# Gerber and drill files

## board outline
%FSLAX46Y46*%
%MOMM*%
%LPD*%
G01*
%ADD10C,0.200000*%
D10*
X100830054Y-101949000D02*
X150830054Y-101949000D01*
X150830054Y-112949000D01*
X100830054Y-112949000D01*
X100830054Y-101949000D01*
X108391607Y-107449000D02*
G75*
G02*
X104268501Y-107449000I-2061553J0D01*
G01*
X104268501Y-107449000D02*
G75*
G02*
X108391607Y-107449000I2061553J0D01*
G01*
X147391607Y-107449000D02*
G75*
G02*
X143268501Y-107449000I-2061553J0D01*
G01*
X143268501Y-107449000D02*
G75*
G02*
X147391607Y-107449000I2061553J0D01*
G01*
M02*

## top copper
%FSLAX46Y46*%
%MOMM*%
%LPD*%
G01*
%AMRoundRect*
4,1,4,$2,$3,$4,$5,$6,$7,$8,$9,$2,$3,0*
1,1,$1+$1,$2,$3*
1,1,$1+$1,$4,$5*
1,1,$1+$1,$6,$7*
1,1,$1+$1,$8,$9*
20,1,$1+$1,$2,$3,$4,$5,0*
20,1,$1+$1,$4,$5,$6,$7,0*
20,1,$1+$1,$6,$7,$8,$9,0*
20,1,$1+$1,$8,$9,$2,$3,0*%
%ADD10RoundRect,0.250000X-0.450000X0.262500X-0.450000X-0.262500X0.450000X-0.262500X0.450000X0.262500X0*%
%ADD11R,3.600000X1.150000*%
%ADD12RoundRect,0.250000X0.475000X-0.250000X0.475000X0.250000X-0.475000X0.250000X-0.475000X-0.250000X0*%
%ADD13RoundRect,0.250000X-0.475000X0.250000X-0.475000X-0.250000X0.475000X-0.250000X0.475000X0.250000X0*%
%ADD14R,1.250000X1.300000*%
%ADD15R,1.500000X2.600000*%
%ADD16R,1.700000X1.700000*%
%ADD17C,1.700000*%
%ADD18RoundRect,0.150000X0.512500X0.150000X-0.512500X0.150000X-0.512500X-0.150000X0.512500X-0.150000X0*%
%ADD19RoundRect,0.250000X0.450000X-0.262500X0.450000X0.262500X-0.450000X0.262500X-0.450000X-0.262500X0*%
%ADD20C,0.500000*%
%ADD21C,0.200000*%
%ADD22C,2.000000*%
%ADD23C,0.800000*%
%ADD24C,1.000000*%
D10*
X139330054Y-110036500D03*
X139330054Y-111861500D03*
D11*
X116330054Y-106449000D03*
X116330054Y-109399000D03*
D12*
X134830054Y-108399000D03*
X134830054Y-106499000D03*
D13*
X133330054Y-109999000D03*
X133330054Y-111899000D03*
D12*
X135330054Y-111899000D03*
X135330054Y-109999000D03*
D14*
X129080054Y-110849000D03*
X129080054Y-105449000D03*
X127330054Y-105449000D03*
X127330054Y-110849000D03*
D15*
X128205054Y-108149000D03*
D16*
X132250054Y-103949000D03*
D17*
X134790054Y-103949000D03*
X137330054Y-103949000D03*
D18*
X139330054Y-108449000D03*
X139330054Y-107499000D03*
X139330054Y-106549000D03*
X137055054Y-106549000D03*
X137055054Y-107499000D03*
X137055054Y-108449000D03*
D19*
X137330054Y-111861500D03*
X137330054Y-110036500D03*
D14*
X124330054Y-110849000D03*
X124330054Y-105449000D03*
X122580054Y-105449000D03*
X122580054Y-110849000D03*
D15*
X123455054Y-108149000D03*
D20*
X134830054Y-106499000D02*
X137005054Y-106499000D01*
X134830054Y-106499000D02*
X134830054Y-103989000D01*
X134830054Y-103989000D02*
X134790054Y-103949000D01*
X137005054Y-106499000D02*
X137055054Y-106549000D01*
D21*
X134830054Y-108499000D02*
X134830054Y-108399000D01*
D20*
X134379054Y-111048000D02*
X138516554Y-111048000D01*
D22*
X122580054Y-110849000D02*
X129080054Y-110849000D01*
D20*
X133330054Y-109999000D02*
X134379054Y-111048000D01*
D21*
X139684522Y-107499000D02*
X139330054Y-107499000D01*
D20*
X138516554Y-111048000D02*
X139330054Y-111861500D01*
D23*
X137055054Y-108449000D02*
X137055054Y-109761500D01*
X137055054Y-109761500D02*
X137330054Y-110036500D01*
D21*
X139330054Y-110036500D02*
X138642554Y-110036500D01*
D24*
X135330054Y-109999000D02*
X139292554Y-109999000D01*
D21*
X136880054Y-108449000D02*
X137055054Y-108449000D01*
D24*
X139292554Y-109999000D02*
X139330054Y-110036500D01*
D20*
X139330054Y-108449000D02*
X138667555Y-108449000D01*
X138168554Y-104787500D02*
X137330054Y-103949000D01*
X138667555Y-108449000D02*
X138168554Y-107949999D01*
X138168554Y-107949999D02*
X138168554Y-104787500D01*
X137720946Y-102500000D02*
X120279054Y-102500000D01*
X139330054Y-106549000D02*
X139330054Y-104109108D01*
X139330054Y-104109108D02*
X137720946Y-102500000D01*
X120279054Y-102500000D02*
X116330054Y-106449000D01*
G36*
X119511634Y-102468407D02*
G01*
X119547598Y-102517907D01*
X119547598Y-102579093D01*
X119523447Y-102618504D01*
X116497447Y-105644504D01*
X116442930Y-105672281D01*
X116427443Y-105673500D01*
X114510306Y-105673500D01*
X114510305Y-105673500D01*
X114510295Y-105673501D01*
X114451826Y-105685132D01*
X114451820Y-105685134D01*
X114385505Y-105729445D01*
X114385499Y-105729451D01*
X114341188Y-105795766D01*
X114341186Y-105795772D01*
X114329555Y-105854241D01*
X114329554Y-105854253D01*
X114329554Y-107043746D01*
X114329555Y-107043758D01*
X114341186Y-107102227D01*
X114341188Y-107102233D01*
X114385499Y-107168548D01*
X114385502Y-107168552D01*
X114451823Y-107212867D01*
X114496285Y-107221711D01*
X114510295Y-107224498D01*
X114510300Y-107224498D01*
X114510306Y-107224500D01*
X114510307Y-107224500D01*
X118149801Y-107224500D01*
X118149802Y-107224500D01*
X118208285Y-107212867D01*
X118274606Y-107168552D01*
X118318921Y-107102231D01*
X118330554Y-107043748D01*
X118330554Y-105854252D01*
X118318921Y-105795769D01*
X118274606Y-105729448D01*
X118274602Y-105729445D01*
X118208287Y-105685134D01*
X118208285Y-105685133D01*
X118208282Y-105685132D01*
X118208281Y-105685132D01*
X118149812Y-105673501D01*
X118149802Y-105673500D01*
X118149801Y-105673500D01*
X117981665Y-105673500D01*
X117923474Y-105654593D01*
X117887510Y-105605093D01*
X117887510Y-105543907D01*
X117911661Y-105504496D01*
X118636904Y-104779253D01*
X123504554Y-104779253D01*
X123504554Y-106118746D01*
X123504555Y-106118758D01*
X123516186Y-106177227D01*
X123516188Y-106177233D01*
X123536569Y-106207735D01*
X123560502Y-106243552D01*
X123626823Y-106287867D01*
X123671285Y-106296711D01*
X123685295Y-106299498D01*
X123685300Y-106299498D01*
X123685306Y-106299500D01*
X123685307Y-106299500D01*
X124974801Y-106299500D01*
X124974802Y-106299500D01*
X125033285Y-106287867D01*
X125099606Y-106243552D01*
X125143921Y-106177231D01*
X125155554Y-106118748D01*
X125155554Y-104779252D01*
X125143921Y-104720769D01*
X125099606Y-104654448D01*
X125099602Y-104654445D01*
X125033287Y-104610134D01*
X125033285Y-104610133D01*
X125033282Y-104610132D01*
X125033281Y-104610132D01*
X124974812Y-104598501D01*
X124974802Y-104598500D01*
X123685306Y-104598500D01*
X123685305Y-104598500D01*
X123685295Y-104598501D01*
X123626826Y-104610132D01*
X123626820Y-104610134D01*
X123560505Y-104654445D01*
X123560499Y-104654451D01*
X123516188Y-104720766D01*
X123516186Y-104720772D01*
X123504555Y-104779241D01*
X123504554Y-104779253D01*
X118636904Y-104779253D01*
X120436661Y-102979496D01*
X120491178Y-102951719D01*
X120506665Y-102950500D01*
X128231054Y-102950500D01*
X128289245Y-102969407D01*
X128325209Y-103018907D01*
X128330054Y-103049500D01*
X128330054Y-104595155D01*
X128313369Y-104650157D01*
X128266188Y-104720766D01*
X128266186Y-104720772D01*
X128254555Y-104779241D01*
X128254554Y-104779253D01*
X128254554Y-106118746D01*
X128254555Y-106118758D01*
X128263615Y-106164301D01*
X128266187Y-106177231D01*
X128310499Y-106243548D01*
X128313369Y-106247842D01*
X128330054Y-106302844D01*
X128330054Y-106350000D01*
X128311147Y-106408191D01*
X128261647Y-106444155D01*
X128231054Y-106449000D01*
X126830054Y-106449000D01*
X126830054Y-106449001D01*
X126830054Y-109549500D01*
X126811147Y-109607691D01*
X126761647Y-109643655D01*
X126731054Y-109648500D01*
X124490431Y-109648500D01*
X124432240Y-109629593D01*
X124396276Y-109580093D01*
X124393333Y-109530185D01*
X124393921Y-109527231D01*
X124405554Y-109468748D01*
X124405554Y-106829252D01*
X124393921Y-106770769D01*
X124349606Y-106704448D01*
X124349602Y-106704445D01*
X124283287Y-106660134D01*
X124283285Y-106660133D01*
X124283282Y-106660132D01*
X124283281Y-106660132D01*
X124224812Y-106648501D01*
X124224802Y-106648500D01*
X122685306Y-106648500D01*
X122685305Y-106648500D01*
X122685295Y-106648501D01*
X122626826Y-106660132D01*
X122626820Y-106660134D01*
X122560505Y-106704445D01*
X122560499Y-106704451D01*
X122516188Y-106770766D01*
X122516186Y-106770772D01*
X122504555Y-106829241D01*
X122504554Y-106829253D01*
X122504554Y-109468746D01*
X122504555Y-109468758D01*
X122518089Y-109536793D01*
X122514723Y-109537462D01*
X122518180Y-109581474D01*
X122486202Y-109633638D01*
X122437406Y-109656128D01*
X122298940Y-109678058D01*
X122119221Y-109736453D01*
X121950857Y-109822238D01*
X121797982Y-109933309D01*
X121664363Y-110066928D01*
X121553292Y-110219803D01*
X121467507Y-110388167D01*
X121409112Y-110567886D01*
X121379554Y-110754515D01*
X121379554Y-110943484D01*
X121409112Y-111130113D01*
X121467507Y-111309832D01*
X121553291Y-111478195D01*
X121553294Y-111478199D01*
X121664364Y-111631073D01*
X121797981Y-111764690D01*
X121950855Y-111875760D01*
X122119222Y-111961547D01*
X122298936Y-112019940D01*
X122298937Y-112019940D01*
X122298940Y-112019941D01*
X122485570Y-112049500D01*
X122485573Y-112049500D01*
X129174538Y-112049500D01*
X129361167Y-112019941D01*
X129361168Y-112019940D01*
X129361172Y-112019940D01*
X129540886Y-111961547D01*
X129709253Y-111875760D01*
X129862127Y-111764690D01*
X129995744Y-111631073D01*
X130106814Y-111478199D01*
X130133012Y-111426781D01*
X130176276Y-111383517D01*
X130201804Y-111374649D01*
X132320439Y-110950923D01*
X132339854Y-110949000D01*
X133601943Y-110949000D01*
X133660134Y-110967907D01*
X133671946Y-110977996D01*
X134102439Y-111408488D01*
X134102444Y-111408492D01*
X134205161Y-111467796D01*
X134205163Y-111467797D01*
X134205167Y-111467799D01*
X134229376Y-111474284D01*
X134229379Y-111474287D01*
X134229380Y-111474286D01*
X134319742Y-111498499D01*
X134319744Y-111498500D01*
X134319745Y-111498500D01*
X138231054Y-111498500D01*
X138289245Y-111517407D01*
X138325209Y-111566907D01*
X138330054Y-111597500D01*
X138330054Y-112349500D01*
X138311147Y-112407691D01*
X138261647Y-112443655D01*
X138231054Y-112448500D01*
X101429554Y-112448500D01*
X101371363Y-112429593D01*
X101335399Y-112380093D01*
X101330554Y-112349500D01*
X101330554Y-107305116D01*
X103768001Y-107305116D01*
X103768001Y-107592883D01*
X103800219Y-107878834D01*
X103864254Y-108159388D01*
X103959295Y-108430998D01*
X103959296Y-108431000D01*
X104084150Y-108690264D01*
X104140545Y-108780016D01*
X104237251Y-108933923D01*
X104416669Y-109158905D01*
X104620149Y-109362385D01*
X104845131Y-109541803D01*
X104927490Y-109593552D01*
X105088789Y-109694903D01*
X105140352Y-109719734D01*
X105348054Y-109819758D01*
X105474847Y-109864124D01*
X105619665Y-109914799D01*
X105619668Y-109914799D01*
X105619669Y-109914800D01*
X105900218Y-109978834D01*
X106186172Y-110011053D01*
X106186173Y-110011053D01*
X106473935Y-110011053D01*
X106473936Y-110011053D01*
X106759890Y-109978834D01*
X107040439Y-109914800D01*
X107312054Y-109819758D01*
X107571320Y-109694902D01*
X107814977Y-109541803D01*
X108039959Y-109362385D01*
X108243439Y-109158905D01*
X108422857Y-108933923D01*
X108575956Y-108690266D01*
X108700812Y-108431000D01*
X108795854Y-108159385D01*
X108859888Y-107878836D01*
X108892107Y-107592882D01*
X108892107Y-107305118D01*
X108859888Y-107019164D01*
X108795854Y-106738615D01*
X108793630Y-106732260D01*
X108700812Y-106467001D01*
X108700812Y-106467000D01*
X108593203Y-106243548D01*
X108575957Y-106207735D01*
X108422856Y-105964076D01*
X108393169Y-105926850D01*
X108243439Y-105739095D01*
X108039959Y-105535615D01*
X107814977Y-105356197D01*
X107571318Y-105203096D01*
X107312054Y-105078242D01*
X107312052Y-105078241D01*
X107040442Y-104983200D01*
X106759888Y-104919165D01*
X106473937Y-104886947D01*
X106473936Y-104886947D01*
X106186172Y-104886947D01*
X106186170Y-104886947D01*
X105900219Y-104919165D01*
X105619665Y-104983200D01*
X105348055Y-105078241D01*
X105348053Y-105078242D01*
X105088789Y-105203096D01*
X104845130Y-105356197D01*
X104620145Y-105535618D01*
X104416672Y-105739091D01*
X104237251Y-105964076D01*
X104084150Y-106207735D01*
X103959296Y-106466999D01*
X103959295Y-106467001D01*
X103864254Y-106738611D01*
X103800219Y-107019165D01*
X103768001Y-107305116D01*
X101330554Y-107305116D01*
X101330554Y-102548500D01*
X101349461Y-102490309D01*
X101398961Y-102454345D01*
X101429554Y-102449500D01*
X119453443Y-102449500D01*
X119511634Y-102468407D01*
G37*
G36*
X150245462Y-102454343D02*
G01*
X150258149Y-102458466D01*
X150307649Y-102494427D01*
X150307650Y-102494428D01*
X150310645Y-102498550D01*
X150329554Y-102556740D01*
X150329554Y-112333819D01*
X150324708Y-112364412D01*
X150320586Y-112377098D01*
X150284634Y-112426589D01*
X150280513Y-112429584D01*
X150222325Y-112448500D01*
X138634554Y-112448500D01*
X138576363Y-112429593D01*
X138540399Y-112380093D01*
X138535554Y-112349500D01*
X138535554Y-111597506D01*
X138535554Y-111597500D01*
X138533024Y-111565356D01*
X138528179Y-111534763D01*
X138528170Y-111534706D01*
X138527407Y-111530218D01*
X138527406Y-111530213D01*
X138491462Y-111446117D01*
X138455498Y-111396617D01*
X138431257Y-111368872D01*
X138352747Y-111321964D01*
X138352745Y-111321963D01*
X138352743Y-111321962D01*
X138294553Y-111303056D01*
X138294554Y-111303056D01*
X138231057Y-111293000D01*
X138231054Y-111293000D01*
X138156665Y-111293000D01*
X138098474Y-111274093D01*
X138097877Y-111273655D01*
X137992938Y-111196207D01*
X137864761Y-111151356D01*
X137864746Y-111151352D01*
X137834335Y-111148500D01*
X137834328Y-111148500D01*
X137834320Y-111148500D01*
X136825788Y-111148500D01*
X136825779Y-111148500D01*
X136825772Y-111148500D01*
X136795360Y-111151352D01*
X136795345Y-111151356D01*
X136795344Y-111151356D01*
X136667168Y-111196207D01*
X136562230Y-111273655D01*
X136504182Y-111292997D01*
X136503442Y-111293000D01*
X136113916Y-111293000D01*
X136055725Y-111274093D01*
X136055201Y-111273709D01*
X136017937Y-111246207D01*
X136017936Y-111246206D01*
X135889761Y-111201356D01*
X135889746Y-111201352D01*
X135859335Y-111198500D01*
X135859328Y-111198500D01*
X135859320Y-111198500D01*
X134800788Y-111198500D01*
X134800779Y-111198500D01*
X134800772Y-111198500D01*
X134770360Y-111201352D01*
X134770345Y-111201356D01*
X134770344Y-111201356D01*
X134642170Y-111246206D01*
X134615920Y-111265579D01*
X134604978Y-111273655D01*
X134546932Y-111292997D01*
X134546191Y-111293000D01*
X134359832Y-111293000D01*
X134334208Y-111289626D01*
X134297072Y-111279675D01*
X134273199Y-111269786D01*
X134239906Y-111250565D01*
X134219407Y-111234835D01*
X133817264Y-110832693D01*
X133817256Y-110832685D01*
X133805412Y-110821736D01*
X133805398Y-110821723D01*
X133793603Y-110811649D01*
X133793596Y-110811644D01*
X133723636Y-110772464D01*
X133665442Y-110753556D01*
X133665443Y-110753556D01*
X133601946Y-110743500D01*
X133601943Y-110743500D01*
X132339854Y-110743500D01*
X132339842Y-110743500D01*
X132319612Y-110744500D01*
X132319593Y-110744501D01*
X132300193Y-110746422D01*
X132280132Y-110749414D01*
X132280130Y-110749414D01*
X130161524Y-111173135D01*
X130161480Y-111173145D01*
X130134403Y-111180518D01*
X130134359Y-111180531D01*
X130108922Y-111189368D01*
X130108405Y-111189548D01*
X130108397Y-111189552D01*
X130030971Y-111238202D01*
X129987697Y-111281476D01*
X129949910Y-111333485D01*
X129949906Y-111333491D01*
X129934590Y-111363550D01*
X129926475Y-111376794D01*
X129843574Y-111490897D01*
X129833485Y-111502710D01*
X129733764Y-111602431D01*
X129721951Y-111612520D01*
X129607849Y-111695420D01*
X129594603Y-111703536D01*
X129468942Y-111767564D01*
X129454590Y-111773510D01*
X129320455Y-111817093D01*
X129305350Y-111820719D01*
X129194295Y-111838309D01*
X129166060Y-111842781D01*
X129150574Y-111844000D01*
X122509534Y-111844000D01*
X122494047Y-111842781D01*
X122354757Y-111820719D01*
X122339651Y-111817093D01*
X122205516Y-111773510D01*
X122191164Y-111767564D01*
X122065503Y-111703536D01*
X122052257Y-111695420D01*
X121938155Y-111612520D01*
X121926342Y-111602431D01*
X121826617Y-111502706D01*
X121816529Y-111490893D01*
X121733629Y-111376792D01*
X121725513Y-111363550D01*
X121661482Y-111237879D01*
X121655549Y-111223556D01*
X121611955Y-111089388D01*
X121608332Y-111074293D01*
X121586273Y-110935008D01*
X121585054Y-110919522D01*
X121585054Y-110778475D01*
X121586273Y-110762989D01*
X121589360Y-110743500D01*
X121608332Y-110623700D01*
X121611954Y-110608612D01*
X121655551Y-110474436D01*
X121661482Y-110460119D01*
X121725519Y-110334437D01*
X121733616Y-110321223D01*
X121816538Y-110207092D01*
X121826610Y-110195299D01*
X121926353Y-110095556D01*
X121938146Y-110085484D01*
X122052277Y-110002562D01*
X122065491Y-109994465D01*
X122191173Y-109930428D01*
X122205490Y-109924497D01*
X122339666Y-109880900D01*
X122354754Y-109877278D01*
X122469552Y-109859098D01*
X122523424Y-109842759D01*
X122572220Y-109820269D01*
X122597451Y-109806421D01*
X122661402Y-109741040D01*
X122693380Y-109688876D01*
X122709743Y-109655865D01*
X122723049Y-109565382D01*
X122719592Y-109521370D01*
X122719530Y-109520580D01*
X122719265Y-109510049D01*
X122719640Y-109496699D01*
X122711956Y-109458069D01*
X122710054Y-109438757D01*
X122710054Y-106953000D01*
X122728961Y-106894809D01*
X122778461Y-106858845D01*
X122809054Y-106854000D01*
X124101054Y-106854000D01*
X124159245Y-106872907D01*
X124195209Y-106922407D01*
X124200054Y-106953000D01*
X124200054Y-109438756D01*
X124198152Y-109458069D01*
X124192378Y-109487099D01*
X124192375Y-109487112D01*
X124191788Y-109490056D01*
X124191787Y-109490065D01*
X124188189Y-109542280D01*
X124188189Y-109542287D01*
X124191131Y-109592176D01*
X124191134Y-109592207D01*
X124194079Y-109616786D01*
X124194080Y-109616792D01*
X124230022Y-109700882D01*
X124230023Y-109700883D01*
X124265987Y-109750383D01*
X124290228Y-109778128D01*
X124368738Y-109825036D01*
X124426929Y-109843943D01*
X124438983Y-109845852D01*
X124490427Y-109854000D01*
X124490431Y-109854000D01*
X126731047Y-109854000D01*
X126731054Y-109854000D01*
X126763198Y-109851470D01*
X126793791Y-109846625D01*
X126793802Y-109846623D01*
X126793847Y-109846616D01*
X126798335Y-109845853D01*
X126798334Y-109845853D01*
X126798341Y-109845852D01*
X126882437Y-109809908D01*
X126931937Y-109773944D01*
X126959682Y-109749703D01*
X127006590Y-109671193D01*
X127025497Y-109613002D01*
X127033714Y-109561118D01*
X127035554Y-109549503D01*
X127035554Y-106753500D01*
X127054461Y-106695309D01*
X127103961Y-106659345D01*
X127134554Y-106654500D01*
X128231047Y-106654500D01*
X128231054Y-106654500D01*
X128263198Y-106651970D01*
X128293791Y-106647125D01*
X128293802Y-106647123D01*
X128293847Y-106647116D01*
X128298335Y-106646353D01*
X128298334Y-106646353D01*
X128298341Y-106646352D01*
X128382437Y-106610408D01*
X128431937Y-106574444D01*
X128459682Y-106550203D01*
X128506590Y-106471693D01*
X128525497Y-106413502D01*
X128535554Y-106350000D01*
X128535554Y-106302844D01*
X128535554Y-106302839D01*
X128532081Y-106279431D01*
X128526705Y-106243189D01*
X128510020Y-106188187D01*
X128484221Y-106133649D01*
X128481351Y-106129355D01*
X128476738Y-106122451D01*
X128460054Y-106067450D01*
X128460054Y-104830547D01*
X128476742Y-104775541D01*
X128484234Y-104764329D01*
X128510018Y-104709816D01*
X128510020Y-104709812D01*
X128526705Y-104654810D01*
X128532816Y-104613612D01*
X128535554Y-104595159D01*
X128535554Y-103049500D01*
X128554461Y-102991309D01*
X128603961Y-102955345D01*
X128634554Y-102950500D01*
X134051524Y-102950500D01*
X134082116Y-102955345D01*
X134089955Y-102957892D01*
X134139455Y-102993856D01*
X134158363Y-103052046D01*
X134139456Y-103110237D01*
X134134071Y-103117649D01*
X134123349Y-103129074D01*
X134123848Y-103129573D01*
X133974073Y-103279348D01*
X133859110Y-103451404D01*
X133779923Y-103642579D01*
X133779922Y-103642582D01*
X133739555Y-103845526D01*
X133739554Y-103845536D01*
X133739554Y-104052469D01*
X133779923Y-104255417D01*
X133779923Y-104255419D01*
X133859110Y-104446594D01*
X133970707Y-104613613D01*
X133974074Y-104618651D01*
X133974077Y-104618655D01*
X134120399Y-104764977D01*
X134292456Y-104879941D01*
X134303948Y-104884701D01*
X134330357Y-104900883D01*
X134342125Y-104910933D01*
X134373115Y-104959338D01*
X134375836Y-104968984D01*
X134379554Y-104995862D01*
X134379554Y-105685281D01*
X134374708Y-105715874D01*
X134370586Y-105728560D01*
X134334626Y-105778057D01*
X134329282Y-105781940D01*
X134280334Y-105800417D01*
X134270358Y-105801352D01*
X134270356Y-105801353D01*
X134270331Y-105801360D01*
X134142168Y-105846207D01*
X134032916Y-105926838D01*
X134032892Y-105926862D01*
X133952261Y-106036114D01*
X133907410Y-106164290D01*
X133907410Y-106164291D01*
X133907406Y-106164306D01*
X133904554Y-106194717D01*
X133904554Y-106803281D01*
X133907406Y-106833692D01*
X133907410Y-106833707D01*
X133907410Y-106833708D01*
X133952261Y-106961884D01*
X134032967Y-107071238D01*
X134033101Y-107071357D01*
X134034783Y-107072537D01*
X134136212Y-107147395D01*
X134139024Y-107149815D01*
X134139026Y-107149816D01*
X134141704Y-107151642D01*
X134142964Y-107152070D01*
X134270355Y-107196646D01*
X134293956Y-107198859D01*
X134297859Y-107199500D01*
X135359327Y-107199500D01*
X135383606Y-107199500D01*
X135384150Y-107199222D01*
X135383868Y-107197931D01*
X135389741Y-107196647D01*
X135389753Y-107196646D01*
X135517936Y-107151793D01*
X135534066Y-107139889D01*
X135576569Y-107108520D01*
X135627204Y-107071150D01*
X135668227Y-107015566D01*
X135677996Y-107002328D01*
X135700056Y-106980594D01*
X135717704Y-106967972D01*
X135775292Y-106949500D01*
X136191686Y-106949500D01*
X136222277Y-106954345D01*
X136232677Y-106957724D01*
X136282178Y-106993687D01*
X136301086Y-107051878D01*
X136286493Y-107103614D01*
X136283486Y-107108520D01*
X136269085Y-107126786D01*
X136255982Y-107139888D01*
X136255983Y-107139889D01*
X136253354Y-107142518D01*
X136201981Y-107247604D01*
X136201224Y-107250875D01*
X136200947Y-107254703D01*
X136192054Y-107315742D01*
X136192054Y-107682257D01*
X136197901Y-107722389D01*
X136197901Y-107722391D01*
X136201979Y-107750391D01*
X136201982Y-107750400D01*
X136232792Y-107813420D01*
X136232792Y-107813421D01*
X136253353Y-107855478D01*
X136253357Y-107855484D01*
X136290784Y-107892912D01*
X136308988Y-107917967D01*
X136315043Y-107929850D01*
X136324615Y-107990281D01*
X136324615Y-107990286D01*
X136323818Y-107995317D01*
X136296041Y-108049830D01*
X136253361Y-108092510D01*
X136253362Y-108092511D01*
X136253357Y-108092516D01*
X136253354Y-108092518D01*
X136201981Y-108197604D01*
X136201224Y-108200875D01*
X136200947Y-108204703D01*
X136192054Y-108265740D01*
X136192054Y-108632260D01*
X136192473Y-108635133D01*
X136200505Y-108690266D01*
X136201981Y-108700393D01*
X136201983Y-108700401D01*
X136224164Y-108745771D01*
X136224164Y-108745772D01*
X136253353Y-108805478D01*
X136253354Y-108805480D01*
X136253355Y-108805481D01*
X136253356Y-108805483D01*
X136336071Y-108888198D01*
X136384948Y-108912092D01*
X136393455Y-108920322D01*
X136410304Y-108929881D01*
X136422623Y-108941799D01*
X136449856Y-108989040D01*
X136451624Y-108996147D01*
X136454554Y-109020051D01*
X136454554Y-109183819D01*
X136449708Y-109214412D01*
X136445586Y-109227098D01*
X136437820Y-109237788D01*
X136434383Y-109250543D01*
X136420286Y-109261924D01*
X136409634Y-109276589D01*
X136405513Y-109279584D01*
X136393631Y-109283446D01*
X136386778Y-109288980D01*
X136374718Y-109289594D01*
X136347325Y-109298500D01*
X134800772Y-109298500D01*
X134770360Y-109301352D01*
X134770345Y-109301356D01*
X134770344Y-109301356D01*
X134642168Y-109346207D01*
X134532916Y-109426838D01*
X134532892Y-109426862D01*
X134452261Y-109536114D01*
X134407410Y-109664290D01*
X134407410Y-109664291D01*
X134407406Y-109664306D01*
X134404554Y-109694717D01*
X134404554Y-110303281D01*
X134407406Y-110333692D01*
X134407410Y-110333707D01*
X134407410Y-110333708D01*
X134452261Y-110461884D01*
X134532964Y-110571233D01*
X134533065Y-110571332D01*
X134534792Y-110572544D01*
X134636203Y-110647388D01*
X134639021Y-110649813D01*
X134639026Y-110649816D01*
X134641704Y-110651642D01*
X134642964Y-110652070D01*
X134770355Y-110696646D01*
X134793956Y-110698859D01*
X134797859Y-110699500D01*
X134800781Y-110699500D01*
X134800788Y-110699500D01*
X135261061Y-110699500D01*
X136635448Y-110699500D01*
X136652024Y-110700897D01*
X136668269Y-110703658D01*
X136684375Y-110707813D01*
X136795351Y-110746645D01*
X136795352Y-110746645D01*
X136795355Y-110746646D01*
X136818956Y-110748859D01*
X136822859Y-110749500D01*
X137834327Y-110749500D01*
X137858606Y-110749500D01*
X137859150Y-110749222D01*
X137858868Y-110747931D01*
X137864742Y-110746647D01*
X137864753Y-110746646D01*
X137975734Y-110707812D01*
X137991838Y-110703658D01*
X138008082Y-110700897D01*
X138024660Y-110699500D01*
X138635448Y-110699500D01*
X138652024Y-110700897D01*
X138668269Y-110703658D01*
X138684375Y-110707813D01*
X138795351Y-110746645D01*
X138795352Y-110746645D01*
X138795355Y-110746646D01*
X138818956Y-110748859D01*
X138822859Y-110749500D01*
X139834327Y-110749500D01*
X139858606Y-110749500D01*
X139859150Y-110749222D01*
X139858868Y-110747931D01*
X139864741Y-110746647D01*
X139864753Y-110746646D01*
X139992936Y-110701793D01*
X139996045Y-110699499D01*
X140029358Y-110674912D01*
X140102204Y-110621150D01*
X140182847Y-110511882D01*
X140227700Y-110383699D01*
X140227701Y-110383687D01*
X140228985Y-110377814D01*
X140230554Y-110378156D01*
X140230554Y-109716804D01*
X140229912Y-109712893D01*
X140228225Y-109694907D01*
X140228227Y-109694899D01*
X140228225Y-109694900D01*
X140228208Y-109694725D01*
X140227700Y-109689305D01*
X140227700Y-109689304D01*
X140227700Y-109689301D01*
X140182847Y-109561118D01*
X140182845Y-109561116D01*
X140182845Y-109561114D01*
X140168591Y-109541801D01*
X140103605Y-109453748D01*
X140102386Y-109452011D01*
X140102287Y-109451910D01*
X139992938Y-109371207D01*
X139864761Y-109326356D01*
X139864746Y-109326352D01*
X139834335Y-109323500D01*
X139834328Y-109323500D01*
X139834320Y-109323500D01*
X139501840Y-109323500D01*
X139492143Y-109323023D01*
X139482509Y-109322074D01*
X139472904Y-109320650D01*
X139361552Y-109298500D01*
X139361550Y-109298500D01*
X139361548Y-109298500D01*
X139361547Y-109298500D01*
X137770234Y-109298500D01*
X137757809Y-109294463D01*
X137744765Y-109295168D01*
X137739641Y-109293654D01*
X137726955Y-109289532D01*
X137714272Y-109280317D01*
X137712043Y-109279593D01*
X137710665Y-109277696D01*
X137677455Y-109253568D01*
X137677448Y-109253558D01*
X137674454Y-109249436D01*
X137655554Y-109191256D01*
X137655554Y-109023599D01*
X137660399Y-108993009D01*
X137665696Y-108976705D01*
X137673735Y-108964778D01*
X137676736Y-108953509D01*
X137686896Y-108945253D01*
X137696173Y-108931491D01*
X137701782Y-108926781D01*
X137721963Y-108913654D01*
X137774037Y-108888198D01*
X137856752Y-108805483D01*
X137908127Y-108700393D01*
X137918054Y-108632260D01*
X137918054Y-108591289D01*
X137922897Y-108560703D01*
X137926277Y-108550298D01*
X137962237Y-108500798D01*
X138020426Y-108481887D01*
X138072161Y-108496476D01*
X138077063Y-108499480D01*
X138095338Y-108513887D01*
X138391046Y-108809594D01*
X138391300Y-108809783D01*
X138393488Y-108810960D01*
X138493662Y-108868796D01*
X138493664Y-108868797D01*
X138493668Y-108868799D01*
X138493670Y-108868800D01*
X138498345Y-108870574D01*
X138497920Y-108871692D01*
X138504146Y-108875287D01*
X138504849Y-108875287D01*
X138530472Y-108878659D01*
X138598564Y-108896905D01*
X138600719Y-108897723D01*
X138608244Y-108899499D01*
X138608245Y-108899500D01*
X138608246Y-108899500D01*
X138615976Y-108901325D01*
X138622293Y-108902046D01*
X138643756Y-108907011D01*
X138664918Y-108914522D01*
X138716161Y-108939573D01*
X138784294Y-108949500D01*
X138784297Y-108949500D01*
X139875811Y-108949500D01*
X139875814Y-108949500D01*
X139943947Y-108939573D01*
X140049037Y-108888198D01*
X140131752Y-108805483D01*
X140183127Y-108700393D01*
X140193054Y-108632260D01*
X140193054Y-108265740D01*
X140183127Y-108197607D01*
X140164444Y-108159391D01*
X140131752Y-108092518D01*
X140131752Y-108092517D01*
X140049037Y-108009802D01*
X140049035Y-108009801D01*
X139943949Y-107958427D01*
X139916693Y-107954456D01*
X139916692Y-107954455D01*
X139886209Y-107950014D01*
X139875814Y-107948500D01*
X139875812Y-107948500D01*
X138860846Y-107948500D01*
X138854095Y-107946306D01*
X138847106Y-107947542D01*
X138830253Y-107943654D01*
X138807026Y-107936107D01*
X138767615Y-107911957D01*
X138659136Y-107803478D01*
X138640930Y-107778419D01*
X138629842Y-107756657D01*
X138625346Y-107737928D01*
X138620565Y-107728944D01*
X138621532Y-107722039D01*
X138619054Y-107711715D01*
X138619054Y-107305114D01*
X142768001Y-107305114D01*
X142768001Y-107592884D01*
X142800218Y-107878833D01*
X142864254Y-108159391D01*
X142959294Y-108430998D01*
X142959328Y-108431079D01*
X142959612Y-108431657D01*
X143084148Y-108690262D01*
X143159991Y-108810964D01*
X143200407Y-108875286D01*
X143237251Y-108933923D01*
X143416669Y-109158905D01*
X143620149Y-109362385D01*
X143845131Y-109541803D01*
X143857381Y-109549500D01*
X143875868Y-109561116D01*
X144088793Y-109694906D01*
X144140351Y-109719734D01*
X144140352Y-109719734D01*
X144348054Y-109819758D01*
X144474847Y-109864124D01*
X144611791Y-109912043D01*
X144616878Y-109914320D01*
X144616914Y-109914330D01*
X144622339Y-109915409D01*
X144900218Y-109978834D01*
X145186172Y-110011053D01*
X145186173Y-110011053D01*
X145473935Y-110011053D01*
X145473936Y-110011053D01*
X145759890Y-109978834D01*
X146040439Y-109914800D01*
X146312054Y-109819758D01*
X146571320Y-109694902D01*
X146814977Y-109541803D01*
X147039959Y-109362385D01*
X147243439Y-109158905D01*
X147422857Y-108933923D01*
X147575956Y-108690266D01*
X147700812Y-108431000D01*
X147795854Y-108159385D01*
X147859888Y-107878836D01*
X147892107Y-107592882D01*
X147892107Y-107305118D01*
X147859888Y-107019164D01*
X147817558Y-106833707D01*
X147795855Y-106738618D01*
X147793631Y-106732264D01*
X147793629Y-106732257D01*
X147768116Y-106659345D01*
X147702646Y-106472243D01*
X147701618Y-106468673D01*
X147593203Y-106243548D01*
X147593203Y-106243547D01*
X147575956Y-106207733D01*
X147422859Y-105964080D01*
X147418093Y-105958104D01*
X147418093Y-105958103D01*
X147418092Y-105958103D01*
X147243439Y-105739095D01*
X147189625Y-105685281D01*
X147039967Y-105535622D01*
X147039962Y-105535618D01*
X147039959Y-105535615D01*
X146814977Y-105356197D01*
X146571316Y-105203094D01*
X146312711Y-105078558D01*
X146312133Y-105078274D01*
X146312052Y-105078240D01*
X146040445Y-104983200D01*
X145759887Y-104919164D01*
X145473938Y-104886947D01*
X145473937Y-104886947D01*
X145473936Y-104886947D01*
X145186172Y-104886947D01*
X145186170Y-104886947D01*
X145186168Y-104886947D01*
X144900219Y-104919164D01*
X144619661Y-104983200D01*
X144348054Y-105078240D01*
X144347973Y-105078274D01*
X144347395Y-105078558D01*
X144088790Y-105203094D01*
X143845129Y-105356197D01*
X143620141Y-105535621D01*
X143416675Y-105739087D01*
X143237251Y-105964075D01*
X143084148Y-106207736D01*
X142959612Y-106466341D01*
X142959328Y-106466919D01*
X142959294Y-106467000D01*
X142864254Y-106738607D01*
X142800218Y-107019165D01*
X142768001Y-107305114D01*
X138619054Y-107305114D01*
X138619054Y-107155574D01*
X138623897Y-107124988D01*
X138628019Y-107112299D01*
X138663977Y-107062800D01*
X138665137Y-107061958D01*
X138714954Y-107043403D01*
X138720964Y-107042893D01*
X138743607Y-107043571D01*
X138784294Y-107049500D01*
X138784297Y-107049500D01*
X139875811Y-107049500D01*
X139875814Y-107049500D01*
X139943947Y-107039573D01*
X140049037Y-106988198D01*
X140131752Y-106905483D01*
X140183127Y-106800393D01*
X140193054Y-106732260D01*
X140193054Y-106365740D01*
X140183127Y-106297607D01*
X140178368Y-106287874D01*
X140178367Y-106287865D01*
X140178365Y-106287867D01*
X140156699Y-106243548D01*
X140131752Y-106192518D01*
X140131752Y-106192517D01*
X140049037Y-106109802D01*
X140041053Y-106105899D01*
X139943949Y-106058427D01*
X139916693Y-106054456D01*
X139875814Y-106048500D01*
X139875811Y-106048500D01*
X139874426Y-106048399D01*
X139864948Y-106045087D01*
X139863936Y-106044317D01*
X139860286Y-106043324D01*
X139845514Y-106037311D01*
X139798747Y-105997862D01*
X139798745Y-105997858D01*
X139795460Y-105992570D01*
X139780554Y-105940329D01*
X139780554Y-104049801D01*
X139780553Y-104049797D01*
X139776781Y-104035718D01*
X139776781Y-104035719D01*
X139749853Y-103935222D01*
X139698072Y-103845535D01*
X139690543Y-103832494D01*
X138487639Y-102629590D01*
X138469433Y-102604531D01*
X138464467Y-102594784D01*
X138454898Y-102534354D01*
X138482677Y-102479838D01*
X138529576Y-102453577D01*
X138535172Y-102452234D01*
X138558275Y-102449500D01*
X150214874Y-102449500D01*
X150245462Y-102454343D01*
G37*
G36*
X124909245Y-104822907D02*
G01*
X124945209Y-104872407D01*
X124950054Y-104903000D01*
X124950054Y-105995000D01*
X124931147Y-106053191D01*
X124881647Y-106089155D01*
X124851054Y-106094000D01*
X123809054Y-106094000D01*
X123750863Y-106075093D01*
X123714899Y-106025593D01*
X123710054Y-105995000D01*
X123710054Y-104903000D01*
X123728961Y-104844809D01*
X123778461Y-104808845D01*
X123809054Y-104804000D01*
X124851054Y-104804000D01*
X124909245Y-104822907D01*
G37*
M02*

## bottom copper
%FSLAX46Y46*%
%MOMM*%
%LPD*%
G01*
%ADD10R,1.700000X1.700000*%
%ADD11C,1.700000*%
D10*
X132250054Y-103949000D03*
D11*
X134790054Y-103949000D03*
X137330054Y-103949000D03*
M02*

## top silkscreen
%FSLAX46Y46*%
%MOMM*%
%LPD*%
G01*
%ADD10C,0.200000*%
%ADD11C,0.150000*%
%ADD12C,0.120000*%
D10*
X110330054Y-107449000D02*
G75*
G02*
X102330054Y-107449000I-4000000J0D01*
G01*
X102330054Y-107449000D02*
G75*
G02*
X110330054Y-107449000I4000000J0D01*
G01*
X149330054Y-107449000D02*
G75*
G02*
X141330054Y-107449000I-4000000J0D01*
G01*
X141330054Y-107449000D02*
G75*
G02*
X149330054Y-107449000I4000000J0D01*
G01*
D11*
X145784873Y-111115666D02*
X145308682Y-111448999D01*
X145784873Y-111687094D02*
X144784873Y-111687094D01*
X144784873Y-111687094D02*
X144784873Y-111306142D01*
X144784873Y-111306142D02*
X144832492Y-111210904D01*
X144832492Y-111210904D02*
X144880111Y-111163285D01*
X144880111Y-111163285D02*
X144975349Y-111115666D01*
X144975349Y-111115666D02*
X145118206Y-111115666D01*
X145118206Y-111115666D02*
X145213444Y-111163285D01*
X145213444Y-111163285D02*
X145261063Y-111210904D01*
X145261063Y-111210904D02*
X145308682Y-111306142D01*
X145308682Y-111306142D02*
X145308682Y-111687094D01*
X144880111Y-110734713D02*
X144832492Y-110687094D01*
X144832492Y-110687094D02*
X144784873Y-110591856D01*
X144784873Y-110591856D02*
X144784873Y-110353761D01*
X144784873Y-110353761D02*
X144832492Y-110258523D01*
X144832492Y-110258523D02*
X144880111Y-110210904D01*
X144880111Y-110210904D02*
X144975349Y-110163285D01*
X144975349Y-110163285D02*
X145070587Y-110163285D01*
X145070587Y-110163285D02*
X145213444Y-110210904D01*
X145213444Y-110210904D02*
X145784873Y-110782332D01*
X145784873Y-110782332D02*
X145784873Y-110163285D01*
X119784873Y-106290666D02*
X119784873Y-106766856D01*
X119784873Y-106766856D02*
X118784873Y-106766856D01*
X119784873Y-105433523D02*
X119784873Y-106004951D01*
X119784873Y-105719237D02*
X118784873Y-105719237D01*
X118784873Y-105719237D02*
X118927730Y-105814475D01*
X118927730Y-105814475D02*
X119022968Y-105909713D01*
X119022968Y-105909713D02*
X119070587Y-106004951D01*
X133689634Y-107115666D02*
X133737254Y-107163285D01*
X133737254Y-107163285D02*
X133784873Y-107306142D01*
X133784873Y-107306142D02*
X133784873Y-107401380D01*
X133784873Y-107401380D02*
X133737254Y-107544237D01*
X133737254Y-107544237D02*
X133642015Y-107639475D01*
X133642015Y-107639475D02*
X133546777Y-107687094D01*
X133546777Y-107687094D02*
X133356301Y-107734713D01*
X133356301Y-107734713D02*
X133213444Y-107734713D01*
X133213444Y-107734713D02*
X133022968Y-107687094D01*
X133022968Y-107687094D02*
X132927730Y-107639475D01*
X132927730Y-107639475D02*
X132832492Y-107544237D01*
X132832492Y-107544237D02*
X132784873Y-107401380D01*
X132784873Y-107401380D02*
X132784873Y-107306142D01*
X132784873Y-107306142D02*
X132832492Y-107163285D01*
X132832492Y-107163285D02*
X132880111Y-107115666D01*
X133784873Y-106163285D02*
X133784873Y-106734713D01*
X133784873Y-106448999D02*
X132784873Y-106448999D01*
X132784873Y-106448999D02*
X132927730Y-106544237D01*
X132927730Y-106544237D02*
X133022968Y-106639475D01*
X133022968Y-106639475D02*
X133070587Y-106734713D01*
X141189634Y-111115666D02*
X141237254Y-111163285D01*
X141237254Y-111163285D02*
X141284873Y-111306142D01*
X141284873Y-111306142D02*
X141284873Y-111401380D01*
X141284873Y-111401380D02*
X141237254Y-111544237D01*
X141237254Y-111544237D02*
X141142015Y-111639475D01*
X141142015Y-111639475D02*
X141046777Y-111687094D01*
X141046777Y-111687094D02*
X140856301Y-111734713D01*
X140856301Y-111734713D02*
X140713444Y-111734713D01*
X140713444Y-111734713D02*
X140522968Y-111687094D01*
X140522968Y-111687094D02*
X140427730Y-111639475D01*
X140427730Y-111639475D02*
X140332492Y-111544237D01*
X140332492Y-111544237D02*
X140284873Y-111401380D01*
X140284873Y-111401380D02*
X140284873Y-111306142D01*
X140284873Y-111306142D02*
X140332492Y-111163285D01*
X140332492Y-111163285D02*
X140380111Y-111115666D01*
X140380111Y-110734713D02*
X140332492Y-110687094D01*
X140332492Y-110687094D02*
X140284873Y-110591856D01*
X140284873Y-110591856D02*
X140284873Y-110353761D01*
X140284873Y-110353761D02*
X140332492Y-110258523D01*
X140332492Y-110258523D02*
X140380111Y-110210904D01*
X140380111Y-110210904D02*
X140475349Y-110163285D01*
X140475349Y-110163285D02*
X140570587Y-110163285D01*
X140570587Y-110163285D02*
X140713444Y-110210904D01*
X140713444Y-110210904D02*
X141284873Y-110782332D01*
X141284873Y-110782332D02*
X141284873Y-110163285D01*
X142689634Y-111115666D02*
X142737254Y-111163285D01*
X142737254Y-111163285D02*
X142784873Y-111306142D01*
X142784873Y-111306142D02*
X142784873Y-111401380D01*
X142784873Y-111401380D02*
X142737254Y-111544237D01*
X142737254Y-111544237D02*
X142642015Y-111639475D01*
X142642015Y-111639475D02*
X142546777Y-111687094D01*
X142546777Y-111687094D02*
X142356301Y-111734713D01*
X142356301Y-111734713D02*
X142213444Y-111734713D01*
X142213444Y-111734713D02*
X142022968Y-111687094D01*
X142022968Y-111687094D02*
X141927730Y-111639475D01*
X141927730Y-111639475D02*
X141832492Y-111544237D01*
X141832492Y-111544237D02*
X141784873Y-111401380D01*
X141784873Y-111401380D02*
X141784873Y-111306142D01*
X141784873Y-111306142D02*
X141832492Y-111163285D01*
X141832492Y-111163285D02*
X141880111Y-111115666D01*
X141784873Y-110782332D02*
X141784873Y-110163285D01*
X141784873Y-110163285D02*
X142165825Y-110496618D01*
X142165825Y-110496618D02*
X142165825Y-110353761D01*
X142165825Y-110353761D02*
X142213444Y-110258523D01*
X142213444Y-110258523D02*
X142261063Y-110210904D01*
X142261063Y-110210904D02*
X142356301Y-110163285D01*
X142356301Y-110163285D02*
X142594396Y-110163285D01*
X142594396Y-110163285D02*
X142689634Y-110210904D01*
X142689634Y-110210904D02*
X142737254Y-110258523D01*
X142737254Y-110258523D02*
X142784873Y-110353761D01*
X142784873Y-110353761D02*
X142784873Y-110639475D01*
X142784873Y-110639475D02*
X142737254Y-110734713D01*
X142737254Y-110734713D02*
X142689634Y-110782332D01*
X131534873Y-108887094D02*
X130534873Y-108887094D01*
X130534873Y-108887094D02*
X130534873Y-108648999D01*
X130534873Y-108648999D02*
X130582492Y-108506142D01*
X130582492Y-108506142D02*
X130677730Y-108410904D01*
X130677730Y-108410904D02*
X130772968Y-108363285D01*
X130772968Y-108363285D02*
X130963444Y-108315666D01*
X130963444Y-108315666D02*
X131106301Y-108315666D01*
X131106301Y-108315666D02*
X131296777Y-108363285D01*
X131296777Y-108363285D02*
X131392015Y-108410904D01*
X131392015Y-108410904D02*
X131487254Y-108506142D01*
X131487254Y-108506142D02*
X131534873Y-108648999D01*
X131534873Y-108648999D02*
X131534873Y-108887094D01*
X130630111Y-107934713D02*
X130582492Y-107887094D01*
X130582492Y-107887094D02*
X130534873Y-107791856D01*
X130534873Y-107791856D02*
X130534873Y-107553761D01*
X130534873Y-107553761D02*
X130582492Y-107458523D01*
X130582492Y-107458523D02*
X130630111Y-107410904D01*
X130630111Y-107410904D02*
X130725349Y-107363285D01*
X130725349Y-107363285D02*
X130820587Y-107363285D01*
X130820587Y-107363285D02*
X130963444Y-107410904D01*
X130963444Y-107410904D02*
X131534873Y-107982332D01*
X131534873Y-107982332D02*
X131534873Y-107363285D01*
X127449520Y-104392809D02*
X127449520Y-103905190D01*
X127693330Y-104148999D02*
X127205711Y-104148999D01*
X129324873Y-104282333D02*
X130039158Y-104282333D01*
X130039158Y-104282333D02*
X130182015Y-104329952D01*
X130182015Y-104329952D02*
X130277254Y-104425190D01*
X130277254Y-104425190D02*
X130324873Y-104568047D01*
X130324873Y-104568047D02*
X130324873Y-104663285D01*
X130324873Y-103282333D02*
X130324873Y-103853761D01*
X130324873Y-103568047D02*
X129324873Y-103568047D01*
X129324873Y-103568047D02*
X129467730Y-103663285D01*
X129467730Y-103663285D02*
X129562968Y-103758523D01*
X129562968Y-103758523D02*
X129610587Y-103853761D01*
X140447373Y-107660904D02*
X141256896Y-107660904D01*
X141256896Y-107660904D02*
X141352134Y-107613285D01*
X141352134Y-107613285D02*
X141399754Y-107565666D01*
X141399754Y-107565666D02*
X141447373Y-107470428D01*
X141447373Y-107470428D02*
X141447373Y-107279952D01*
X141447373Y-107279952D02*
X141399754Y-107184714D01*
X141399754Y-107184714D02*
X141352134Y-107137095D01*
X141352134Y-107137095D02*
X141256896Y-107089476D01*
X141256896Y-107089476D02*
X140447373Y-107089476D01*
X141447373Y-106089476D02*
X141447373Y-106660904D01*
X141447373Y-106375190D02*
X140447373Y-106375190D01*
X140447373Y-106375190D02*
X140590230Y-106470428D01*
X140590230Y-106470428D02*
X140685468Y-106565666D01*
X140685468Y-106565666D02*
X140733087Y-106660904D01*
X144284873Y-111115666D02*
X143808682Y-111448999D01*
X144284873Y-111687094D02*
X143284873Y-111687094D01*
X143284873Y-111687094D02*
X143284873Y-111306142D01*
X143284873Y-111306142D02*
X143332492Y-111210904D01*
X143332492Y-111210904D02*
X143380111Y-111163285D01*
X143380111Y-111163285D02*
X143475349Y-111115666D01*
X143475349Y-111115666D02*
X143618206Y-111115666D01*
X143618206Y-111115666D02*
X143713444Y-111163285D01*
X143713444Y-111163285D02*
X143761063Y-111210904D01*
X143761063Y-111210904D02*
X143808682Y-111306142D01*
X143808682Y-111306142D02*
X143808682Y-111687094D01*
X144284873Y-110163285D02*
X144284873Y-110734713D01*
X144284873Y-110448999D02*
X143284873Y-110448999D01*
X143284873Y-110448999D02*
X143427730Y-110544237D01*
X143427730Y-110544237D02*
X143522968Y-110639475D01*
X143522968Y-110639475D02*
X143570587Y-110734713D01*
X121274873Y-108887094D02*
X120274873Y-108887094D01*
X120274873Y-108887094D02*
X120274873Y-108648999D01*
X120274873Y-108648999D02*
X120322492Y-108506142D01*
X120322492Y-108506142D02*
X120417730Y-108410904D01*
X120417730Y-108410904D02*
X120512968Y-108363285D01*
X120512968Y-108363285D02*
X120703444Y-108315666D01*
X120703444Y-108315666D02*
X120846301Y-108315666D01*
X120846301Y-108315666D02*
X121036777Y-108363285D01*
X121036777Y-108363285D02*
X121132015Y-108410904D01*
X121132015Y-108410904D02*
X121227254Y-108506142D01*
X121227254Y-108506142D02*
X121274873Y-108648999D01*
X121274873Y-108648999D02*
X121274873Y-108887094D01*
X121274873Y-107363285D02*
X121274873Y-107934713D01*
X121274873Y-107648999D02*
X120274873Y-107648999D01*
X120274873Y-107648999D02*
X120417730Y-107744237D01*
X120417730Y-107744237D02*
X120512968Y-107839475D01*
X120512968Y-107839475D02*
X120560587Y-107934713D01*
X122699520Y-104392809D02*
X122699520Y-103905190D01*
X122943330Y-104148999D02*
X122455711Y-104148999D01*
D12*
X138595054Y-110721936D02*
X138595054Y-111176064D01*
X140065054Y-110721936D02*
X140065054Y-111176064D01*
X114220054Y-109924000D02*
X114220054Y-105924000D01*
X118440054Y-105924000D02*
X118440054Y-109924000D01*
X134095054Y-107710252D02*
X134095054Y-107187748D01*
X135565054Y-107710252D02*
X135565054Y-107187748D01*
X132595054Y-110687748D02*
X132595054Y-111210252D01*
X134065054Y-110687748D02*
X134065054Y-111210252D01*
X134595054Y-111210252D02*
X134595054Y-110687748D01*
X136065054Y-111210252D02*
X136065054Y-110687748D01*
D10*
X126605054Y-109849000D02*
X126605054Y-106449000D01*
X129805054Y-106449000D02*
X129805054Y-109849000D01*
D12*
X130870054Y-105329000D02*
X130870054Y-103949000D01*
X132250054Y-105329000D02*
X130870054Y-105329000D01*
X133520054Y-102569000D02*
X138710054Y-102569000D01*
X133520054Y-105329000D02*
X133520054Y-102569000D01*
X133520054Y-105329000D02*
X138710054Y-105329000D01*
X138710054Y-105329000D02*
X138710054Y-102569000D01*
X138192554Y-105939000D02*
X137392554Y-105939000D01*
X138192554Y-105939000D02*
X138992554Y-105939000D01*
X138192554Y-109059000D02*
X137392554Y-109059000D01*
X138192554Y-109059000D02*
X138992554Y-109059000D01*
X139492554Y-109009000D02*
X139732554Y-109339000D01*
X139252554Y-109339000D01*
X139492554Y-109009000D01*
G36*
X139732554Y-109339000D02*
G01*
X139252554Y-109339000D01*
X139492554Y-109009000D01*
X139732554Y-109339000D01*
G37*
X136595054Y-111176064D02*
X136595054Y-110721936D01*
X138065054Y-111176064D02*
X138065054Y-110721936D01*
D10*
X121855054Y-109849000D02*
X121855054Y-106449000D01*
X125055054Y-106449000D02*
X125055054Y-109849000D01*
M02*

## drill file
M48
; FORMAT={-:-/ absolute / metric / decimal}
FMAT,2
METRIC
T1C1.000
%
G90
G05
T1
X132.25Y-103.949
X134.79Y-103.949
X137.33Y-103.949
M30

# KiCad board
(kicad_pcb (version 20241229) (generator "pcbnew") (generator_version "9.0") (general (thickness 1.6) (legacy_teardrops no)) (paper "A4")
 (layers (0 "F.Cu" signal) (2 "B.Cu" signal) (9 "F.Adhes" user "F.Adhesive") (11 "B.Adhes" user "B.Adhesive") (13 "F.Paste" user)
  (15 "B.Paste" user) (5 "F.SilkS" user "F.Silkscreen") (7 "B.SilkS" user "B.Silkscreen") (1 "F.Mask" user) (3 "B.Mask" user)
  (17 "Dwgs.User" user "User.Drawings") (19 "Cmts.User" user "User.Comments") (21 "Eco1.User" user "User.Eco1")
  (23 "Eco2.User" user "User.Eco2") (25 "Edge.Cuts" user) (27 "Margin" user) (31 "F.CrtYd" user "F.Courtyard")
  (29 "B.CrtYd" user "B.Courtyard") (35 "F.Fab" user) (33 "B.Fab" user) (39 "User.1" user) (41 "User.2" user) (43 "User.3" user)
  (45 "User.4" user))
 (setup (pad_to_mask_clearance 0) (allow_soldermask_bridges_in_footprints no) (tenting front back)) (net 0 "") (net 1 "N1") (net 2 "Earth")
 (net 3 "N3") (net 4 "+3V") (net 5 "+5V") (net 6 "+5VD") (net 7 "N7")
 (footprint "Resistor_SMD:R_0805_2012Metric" (layer "F.Cu") (at 139.330054 110.949 -90)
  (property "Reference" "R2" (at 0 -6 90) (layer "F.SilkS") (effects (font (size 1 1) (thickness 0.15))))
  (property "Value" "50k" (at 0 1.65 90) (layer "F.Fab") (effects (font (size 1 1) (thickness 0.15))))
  (fp_line (start -0.227064 0.735) (end 0.227064 0.735) (stroke (width 0.12) (type solid)) (layer "F.SilkS"))
  (fp_line (start -0.227064 -0.735) (end 0.227064 -0.735) (stroke (width 0.12) (type solid)) (layer "F.SilkS"))
  (pad "1" smd roundrect (at -0.9125 0 270) (size 1.025 1.4) (layers "F.Cu" "F.Mask" "F.Paste") (roundrect_rratio 0.243902) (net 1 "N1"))
  (pad "2" smd roundrect (at 0.9125 0 270) (size 1.025 1.4) (layers "F.Cu" "F.Mask" "F.Paste") (roundrect_rratio 0.243902) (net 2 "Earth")))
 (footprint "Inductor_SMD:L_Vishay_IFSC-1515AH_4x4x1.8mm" (layer "F.Cu") (at 116.330054 107.924 -90)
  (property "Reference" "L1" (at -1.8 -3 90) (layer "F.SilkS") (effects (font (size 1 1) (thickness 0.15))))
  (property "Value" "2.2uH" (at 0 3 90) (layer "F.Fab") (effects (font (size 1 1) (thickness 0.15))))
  (fp_line (start 2 2.11) (end -2 2.11) (stroke (width 0.12) (type solid)) (layer "F.SilkS"))
  (fp_line (start -2 -2.11) (end 2 -2.11) (stroke (width 0.12) (type solid)) (layer "F.SilkS"))
  (pad "1" smd rect (at -1.475 0 270) (size 1.15 3.6) (layers "F.Cu" "F.Mask" "F.Paste") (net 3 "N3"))
  (pad "2" smd rect (at 1.475 0 270) (size 1.15 3.6) (layers "F.Cu" "F.Mask" "F.Paste") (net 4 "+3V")))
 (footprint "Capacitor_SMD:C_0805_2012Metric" (layer "F.Cu") (at 134.830054 107.449 90)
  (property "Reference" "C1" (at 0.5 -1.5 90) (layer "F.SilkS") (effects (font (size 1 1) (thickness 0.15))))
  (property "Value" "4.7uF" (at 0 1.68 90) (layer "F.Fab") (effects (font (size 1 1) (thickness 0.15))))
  (fp_line (start -0.261252 -0.735) (end 0.261252 -0.735) (stroke (width 0.12) (type solid)) (layer "F.SilkS"))
  (fp_line (start -0.261252 0.735) (end 0.261252 0.735) (stroke (width 0.12) (type solid)) (layer "F.SilkS"))
  (pad "1" smd roundrect (at -0.95 0 90) (size 1 1.45) (layers "F.Cu" "F.Mask" "F.Paste") (roundrect_rratio 0.25) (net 2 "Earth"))
  (pad "2" smd roundrect (at 0.95 0 90) (size 1 1.45) (layers "F.Cu" "F.Mask" "F.Paste") (roundrect_rratio 0.25) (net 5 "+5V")))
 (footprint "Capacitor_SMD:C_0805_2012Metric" (layer "F.Cu") (at 133.330054 110.949 -90)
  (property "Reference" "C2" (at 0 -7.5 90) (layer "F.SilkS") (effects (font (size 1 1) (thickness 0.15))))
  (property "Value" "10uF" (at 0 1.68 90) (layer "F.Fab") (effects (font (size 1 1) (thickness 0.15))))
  (fp_line (start -0.261252 0.735) (end 0.261252 0.735) (stroke (width 0.12) (type solid)) (layer "F.SilkS"))
  (fp_line (start -0.261252 -0.735) (end 0.261252 -0.735) (stroke (width 0.12) (type solid)) (layer "F.SilkS"))
  (pad "1" smd roundrect (at -0.95 0 270) (size 1 1.45) (layers "F.Cu" "F.Mask" "F.Paste") (roundrect_rratio 0.25) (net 2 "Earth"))
  (pad "2" smd roundrect (at 0.95 0 270) (size 1 1.45) (layers "F.Cu" "F.Mask" "F.Paste") (roundrect_rratio 0.25) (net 4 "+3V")))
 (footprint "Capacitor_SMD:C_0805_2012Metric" (layer "F.Cu") (at 135.330054 110.949 90)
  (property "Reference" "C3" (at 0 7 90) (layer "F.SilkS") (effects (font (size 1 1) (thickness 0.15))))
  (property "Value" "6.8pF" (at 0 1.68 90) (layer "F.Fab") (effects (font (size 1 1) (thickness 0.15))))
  (fp_line (start -0.261252 -0.735) (end 0.261252 -0.735) (stroke (width 0.12) (type solid)) (layer "F.SilkS"))
  (fp_line (start -0.261252 0.735) (end 0.261252 0.735) (stroke (width 0.12) (type solid)) (layer "F.SilkS"))
  (pad "1" smd roundrect (at -0.95 0 90) (size 1 1.45) (layers "F.Cu" "F.Mask" "F.Paste") (roundrect_rratio 0.25) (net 4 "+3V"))
  (pad "2" smd roundrect (at 0.95 0 90) (size 1 1.45) (layers "F.Cu" "F.Mask" "F.Paste") (roundrect_rratio 0.25) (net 1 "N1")))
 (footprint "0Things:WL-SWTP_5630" (layer "F.Cu") (at 128.205054 108.149 90)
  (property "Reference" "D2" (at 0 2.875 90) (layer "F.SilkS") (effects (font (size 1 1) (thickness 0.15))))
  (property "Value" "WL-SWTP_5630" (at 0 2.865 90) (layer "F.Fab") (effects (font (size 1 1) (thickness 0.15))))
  (fp_line (start -1.7 -1.6) (end 1.7 -1.6) (stroke (width 0.2) (type solid)) (layer "F.SilkS"))
  (fp_line (start 1.7 1.6) (end -1.7 1.6) (stroke (width 0.2) (type solid)) (layer "F.SilkS"))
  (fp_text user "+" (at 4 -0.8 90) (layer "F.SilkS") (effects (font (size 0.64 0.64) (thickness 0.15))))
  (pad "1" smd rect (at -2.7 0.875 90) (size 1.3 1.25) (layers "F.Cu" "F.Mask" "F.Paste") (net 2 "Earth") (solder_mask_margin 0.102))
  (pad "2" smd rect (at 2.7 0.875 90) (size 1.3 1.25) (layers "F.Cu" "F.Mask" "F.Paste") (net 2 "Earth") (solder_mask_margin 0.102))
  (pad "3" smd rect (at 2.7 -0.875 90) (size 1.3 1.25) (layers "F.Cu" "F.Mask" "F.Paste") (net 4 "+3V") (solder_mask_margin 0.102))
  (pad "4" smd rect (at -2.7 -0.875 90) (size 1.3 1.25) (layers "F.Cu" "F.Mask" "F.Paste") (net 2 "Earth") (solder_mask_margin 0.102))
  (pad "5" smd rect (at 0 0 90) (size 2.6 1.5) (layers "F.Cu" "F.Mask" "F.Paste") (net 2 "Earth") (solder_mask_margin 0.102)))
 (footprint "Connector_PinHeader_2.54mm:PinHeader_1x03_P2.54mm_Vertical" (layer "F.Cu") (at 132.250054 103.949 90)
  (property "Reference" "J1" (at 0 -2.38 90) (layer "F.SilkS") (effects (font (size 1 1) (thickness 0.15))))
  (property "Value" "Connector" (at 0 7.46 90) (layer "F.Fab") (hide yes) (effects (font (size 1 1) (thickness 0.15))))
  (fp_line (start -1.38 -1.38) (end 0 -1.38) (stroke (width 0.12) (type solid)) (layer "F.SilkS"))
  (fp_line (start -1.38 0) (end -1.38 -1.38) (stroke (width 0.12) (type solid)) (layer "F.SilkS"))
  (fp_line (start 1.38 1.27) (end 1.38 6.46) (stroke (width 0.12) (type solid)) (layer "F.SilkS"))
  (fp_line (start -1.38 1.27) (end 1.38 1.27) (stroke (width 0.12) (type solid)) (layer "F.SilkS"))
  (fp_line (start -1.38 1.27) (end -1.38 6.46) (stroke (width 0.12) (type solid)) (layer "F.SilkS"))
  (fp_line (start -1.38 6.46) (end 1.38 6.46) (stroke (width 0.12) (type solid)) (layer "F.SilkS"))
  (pad "1" thru_hole rect (at 0 0 90) (size 1.7 1.7) (drill 1) (layers "*.Cu" "*.Mask") (remove_unused_layers no) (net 2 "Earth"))
  (pad "2" thru_hole circle (at 0 2.54 90) (size 1.7 1.7) (drill 1) (layers "*.Cu" "*.Mask") (remove_unused_layers no) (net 5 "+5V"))
  (pad "3" thru_hole circle (at 0 5.08 90) (size 1.7 1.7) (drill 1) (layers "*.Cu" "*.Mask") (remove_unused_layers no) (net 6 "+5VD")))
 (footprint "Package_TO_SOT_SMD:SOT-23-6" (layer "F.Cu") (at 138.192554 107.499 180)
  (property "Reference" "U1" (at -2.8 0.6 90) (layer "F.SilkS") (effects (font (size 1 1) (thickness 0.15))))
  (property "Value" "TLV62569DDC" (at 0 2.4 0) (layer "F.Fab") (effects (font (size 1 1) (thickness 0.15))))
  (fp_line (start 0 1.56) (end 0.8 1.56) (stroke (width 0.12) (type solid)) (layer "F.SilkS"))
  (fp_line (start 0 1.56) (end -0.8 1.56) (stroke (width 0.12) (type solid)) (layer "F.SilkS"))
  (fp_line (start 0 -1.56) (end 0.8 -1.56) (stroke (width 0.12) (type solid)) (layer "F.SilkS"))
  (fp_line (start 0 -1.56) (end -0.8 -1.56) (stroke (width 0.12) (type solid)) (layer "F.SilkS"))
  (fp_poly (pts (xy -1.3 -1.51) (xy -1.54 -1.84) (xy -1.06 -1.84)) (stroke (width 0.12) (type solid)) (fill yes) (layer "F.SilkS"))
  (pad "1" smd roundrect (at -1.1375 -0.95 180) (size 1.325 0.6) (layers "F.Cu" "F.Mask" "F.Paste") (roundrect_rratio 0.25) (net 6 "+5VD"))
  (pad "2" smd roundrect (at -1.1375 0 180) (size 1.325 0.6) (layers "F.Cu" "F.Mask" "F.Paste") (roundrect_rratio 0.25) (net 2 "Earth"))
  (pad "3" smd roundrect (at -1.1375 0.95 180) (size 1.325 0.6) (layers "F.Cu" "F.Mask" "F.Paste") (roundrect_rratio 0.25) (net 3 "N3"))
  (pad "4" smd roundrect (at 1.1375 0.95 180) (size 1.325 0.6) (layers "F.Cu" "F.Mask" "F.Paste") (roundrect_rratio 0.25) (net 5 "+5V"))
  (pad "5" smd roundrect (at 1.1375 0 180) (size 1.325 0.6) (layers "F.Cu" "F.Mask" "F.Paste") (roundrect_rratio 0.25) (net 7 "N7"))
  (pad "6" smd roundrect (at 1.1375 -0.95 180) (size 1.325 0.6) (layers "F.Cu" "F.Mask" "F.Paste") (roundrect_rratio 0.25) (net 1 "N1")))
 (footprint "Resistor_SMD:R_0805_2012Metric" (layer "F.Cu") (at 137.330054 110.949 90)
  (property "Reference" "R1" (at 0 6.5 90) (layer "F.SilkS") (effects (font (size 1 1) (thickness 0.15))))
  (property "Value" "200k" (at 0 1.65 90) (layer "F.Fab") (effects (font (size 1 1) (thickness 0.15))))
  (fp_line (start -0.227064 -0.735) (end 0.227064 -0.735) (stroke (width 0.12) (type solid)) (layer "F.SilkS"))
  (fp_line (start -0.227064 0.735) (end 0.227064 0.735) (stroke (width 0.12) (type solid)) (layer "F.SilkS"))
  (pad "1" smd roundrect (at -0.9125 0 90) (size 1.025 1.4) (layers "F.Cu" "F.Mask" "F.Paste") (roundrect_rratio 0.243902) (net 4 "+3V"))
  (pad "2" smd roundrect (at 0.9125 0 90) (size 1.025 1.4) (layers "F.Cu" "F.Mask" "F.Paste") (roundrect_rratio 0.243902) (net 1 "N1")))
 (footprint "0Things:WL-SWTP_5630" (layer "F.Cu") (at 123.455054 108.149 90)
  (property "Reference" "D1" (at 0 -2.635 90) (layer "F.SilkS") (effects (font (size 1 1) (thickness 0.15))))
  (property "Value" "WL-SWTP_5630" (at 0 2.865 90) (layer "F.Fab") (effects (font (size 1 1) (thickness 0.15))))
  (fp_line (start -1.7 -1.6) (end 1.7 -1.6) (stroke (width 0.2) (type solid)) (layer "F.SilkS"))
  (fp_line (start 1.7 1.6) (end -1.7 1.6) (stroke (width 0.2) (type solid)) (layer "F.SilkS"))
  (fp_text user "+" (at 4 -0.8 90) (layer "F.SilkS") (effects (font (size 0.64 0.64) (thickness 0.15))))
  (pad "1" smd rect (at -2.7 0.875 90) (size 1.3 1.25) (layers "F.Cu" "F.Mask" "F.Paste") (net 2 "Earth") (solder_mask_margin 0.102))
  (pad "2" smd rect (at 2.7 0.875 90) (size 1.3 1.25) (layers "F.Cu" "F.Mask" "F.Paste") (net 2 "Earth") (solder_mask_margin 0.102))
  (pad "3" smd rect (at 2.7 -0.875 90) (size 1.3 1.25) (layers "F.Cu" "F.Mask" "F.Paste") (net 4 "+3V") (solder_mask_margin 0.102))
  (pad "4" smd rect (at -2.7 -0.875 90) (size 1.3 1.25) (layers "F.Cu" "F.Mask" "F.Paste") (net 2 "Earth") (solder_mask_margin 0.102))
  (pad "5" smd rect (at 0 0 90) (size 2.6 1.5) (layers "F.Cu" "F.Mask" "F.Paste") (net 2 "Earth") (solder_mask_margin 0.102)))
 (gr_circle (center 106.330054 107.449) (end 106.330054 103.449) (stroke (width 0.2) (type solid)) (fill no) (layer "F.SilkS"))
 (gr_circle (center 145.330054 107.449) (end 145.330054 103.449) (stroke (width 0.2) (type solid)) (fill no) (layer "F.SilkS"))
 (gr_rect (start 100.830054 101.949) (end 150.830054 112.949) (stroke (width 0.2) (type solid)) (fill no) (layer "Edge.Cuts"))
 (gr_circle (center 106.330054 107.449) (end 108.330054 107.949) (stroke (width 0.2) (type solid)) (fill no) (layer "Edge.Cuts"))
 (gr_circle (center 145.330054 107.449) (end 147.330054 106.949) (stroke (width 0.2) (type solid)) (fill no) (layer "Edge.Cuts"))
 (segment (start 134.830054 106.499) (end 137.005054 106.499) (width 0.5) (layer "F.Cu") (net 5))
 (segment (start 134.830054 106.499) (end 134.830054 103.989) (width 0.5) (layer "F.Cu") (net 5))
 (segment (start 134.830054 103.989) (end 134.790054 103.949) (width 0.5) (layer "F.Cu") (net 5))
 (segment (start 137.005054 106.499) (end 137.055054 106.549) (width 0.5) (layer "F.Cu") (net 5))
 (segment (start 134.830054 108.499) (end 134.830054 108.399) (width 0.2) (layer "F.Cu") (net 2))
 (segment (start 134.379054 111.048) (end 138.516554 111.048) (width 0.5) (layer "F.Cu") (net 2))
 (segment (start 122.580054 110.849) (end 129.080054 110.849) (width 2) (layer "F.Cu") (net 2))
 (segment (start 133.330054 109.999) (end 134.379054 111.048) (width 0.5) (layer "F.Cu") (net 2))
 (segment (start 139.684522 107.499) (end 139.330054 107.499) (width 0.2) (layer "F.Cu") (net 2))
 (segment (start 138.516554 111.048) (end 139.330054 111.8615) (width 0.5) (layer "F.Cu") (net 2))
 (segment (start 137.055054 108.449) (end 137.055054 109.7615) (width 0.8) (layer "F.Cu") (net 1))
 (segment (start 137.055054 109.7615) (end 137.330054 110.0365) (width 0.8) (layer "F.Cu") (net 1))
 (segment (start 139.330054 110.0365) (end 138.642554 110.0365) (width 0.2) (layer "F.Cu") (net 1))
 (segment (start 135.330054 109.999) (end 139.292554 109.999) (width 1) (layer "F.Cu") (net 1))
 (segment (start 136.880054 108.449) (end 137.055054 108.449) (width 0.2) (layer "F.Cu") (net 1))
 (segment (start 139.292554 109.999) (end 139.330054 110.0365) (width 1) (layer "F.Cu") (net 1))
 (segment (start 139.330054 108.449) (end 138.667555 108.449) (width 0.5) (layer "F.Cu") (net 6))
 (segment (start 138.168554 104.7875) (end 137.330054 103.949) (width 0.5) (layer "F.Cu") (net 6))
 (segment (start 138.667555 108.449) (end 138.168554 107.949999) (width 0.5) (layer "F.Cu") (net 6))
 (segment (start 138.168554 107.949999) (end 138.168554 104.7875) (width 0.5) (layer "F.Cu") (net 6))
 (segment (start 137.720946 102.5) (end 120.279054 102.5) (width 0.5) (layer "F.Cu") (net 3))
 (segment (start 139.330054 106.549) (end 139.330054 104.109108) (width 0.5) (layer "F.Cu") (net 3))
 (segment (start 139.330054 104.109108) (end 137.720946 102.5) (width 0.5) (layer "F.Cu") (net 3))
 (segment (start 120.279054 102.5) (end 116.330054 106.449) (width 0.5) (layer "F.Cu") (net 3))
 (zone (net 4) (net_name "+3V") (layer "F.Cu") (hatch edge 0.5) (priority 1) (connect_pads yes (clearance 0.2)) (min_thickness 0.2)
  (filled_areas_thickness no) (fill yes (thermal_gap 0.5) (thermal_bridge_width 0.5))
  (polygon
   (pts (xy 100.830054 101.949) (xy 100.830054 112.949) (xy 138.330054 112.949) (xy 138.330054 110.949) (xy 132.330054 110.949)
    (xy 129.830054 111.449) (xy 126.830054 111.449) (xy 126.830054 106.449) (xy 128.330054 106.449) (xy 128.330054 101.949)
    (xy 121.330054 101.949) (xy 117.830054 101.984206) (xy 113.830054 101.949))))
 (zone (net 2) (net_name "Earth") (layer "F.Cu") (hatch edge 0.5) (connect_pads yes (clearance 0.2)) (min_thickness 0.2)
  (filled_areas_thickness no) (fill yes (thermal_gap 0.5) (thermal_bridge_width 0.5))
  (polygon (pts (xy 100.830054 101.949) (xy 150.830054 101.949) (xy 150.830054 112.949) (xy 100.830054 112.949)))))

